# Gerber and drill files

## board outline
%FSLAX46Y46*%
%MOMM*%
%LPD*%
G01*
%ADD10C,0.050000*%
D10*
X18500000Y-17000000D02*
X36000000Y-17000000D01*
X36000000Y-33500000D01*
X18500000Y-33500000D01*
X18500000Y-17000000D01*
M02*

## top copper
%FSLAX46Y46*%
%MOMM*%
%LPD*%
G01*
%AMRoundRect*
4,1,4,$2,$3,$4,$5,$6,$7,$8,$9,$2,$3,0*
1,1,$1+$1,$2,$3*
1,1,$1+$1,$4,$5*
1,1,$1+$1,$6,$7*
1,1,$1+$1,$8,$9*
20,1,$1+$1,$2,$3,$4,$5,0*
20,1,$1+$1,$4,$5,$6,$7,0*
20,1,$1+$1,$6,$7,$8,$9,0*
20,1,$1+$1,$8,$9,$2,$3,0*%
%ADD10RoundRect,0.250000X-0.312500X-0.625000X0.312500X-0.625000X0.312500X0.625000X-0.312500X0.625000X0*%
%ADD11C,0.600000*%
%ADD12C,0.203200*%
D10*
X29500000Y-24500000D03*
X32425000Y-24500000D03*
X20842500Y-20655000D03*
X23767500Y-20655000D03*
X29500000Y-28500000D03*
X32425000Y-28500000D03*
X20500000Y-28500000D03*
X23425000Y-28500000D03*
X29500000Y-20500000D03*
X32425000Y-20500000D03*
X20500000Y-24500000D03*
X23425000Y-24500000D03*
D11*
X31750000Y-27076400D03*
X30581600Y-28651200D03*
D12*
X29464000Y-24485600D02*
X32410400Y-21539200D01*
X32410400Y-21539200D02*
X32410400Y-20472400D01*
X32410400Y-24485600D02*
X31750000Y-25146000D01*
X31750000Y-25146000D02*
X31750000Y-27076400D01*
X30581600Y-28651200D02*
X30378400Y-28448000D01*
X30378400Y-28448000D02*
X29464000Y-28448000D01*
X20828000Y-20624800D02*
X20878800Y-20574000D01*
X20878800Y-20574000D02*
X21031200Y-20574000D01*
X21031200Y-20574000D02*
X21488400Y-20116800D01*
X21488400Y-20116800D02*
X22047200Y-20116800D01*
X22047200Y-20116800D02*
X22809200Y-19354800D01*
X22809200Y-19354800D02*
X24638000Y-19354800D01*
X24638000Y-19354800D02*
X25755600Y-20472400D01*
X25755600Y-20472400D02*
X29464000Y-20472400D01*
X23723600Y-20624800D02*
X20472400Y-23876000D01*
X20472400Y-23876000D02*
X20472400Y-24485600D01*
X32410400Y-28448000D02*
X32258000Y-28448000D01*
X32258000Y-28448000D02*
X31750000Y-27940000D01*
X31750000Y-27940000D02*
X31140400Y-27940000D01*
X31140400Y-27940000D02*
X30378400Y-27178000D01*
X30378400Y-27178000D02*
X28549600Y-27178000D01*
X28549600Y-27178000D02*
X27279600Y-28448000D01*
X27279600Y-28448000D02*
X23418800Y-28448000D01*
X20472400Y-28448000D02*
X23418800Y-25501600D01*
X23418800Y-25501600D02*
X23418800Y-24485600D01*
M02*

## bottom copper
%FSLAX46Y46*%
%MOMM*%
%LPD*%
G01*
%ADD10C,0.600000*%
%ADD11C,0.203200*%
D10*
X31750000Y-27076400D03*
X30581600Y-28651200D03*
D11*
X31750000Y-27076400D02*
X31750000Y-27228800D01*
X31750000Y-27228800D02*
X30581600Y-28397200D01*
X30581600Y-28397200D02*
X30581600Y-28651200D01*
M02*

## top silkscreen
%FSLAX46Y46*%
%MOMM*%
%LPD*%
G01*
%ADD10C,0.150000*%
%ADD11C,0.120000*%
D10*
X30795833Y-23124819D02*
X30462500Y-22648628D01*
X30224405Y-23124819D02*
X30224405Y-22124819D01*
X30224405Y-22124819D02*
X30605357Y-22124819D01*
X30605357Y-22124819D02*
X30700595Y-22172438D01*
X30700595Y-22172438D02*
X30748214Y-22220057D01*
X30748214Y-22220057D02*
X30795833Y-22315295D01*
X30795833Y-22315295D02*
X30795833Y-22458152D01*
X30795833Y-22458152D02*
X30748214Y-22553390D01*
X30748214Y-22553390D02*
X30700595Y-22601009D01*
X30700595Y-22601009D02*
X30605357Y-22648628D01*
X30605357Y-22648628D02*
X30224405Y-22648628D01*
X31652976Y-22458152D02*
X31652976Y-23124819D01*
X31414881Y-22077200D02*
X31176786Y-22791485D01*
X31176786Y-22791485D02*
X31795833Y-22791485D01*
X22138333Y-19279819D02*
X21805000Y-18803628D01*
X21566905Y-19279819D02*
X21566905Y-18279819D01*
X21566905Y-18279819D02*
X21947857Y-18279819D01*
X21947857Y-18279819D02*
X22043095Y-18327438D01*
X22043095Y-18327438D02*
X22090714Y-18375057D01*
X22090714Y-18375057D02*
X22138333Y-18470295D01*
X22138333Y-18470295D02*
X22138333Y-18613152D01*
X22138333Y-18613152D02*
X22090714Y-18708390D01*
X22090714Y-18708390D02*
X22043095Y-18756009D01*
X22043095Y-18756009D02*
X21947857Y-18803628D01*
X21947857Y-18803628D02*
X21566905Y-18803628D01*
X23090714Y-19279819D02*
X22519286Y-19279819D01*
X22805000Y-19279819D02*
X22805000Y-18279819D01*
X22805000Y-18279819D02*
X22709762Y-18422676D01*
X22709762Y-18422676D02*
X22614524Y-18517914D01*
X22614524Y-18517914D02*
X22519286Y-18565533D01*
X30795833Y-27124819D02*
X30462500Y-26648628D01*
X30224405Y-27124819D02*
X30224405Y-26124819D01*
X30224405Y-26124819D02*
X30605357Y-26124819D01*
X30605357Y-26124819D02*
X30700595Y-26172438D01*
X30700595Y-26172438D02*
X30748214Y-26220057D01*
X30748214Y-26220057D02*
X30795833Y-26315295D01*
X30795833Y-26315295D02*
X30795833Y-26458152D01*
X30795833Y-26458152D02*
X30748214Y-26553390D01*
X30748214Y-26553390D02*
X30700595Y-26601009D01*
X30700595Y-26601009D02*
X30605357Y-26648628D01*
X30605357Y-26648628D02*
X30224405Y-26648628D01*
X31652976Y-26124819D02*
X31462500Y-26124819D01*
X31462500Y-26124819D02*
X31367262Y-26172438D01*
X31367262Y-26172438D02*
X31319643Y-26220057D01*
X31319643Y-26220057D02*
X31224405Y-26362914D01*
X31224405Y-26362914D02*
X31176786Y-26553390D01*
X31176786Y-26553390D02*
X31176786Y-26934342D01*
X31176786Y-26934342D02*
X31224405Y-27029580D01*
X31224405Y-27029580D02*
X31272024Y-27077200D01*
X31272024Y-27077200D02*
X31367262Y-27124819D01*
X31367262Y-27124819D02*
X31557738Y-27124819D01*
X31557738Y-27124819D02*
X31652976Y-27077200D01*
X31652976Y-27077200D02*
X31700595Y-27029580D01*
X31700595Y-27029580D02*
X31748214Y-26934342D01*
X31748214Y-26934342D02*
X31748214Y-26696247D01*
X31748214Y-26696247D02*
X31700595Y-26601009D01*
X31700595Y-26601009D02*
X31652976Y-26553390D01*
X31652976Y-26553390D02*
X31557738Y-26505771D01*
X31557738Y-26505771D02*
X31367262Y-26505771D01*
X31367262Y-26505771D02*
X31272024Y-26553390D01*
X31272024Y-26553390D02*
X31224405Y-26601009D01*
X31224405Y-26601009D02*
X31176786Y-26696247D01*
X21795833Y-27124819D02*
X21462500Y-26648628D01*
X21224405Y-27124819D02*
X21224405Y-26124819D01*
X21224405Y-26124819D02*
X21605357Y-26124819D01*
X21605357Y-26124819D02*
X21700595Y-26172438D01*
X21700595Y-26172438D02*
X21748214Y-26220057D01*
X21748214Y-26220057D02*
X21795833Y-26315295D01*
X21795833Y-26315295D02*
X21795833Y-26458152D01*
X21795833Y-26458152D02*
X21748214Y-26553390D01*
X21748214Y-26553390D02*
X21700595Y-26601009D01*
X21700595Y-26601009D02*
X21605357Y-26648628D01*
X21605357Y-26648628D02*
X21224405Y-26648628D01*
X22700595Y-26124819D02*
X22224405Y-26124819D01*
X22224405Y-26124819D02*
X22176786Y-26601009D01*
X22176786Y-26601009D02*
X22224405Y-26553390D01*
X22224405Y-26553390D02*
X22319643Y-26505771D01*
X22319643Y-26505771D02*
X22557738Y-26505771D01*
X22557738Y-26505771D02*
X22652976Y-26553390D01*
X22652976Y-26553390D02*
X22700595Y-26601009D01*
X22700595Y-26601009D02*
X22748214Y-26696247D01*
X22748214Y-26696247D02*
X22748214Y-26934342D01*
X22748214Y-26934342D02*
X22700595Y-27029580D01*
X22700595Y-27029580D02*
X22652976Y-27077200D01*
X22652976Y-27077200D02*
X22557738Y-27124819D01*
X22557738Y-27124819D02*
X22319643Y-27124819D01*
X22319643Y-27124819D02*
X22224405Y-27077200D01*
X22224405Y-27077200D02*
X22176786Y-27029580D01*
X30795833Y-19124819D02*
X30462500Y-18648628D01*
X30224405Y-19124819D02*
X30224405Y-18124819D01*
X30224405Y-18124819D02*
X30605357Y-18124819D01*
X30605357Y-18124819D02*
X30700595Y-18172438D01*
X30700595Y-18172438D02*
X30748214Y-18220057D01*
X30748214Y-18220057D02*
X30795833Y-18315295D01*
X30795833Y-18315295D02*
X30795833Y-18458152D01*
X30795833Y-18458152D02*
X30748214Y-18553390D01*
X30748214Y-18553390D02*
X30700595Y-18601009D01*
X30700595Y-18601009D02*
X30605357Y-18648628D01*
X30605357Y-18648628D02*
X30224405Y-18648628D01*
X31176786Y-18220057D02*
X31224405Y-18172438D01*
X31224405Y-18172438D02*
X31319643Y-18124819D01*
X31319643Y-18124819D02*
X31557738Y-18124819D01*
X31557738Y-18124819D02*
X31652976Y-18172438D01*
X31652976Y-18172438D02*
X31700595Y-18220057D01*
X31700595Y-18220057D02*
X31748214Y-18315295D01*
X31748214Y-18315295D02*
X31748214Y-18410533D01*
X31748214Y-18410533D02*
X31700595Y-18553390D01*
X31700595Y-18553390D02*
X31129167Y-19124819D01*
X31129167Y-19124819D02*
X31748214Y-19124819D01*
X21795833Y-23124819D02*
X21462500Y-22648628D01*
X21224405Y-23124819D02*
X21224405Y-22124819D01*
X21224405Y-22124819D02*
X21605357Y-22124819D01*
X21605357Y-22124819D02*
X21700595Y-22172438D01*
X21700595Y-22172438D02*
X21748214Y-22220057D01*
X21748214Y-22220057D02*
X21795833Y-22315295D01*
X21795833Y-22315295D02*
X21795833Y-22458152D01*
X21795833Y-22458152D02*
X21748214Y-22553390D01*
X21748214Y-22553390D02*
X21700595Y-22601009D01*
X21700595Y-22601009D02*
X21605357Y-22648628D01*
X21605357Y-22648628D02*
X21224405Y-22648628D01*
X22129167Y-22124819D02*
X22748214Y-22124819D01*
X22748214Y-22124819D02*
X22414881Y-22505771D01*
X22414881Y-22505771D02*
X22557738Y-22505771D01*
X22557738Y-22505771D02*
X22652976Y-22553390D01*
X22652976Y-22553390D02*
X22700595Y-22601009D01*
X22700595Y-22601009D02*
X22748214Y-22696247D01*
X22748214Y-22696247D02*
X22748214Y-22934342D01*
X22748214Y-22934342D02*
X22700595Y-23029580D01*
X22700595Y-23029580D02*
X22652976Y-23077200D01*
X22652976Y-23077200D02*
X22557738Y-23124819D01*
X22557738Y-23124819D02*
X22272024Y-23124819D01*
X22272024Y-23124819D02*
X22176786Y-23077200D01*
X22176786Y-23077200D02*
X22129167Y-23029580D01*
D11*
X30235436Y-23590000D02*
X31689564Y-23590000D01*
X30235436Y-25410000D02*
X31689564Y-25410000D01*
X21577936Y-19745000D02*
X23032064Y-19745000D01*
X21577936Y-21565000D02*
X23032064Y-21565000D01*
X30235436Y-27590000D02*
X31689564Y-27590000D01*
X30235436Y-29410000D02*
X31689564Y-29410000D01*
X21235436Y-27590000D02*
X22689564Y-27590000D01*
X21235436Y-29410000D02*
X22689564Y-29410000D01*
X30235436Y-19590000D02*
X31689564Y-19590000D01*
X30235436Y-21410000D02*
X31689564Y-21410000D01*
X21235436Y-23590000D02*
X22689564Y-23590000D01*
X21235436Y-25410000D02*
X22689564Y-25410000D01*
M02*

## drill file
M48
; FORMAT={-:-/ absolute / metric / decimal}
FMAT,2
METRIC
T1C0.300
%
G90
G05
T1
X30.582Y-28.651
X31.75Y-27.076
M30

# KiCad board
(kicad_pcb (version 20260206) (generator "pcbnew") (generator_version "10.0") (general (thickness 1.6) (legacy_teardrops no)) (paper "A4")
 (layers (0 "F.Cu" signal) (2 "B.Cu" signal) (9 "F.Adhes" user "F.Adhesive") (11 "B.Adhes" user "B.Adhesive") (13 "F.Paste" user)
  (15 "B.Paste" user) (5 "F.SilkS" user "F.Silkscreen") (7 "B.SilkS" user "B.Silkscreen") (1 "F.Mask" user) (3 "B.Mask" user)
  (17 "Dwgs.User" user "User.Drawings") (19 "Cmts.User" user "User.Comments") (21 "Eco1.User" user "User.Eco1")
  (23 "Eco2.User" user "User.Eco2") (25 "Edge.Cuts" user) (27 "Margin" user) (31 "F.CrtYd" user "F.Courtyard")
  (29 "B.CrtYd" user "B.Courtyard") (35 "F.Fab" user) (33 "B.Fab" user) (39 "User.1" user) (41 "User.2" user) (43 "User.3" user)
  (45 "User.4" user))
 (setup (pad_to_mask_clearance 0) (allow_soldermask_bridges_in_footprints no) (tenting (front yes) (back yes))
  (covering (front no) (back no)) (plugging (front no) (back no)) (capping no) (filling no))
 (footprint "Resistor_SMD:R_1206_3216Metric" (layer "F.Cu") (at 30.9625 24.5)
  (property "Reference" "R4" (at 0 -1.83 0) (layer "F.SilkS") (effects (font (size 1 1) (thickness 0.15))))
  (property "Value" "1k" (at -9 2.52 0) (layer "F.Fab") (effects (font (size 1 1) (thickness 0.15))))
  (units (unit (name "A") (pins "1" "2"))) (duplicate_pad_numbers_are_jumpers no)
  (fp_line (start -0.727064 -0.91) (end 0.727064 -0.91) (stroke (width 0.12) (type solid)) (layer "F.SilkS"))
  (fp_line (start -0.727064 0.91) (end 0.727064 0.91) (stroke (width 0.12) (type solid)) (layer "F.SilkS"))
  (pad "1" smd roundrect (at -1.4625 0) (size 1.125 1.75) (layers "F.Cu" "F.Mask" "F.Paste") (roundrect_rratio 0.222222)
   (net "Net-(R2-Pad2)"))
  (pad "2" smd roundrect (at 1.4625 0) (size 1.125 1.75) (layers "F.Cu" "F.Mask" "F.Paste") (roundrect_rratio 0.222222)
   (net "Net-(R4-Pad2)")))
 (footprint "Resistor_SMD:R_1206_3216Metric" (layer "F.Cu") (at 22.305 20.655)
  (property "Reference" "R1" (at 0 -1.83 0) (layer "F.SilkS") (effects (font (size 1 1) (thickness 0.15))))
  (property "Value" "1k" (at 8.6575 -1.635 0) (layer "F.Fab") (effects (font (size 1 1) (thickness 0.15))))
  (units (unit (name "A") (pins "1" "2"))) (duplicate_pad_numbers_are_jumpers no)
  (fp_line (start -0.727064 -0.91) (end 0.727064 -0.91) (stroke (width 0.12) (type solid)) (layer "F.SilkS"))
  (fp_line (start -0.727064 0.91) (end 0.727064 0.91) (stroke (width 0.12) (type solid)) (layer "F.SilkS"))
  (pad "1" smd roundrect (at -1.4625 0) (size 1.125 1.75) (layers "F.Cu" "F.Mask" "F.Paste") (roundrect_rratio 0.222222)
   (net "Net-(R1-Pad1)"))
  (pad "2" smd roundrect (at 1.4625 0) (size 1.125 1.75) (layers "F.Cu" "F.Mask" "F.Paste") (roundrect_rratio 0.222222)
   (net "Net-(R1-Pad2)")))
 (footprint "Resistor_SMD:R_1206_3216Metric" (layer "F.Cu") (at 30.9625 28.5)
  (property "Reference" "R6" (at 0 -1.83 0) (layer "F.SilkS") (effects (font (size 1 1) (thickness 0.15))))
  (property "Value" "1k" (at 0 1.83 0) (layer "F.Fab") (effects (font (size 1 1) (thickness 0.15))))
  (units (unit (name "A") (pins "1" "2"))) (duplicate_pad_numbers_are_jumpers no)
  (fp_line (start -0.727064 -0.91) (end 0.727064 -0.91) (stroke (width 0.12) (type solid)) (layer "F.SilkS"))
  (fp_line (start -0.727064 0.91) (end 0.727064 0.91) (stroke (width 0.12) (type solid)) (layer "F.SilkS"))
  (pad "1" smd roundrect (at -1.4625 0) (size 1.125 1.75) (layers "F.Cu" "F.Mask" "F.Paste") (roundrect_rratio 0.222222)
   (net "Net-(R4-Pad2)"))
  (pad "2" smd roundrect (at 1.4625 0) (size 1.125 1.75) (layers "F.Cu" "F.Mask" "F.Paste") (roundrect_rratio 0.222222)
   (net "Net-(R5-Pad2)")))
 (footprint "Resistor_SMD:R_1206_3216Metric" (layer "F.Cu") (at 21.9625 28.5)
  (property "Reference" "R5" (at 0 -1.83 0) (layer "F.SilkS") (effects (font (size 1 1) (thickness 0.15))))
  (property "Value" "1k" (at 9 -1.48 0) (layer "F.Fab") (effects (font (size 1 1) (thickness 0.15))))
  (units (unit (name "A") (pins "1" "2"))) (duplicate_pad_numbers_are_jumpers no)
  (fp_line (start -0.727064 -0.91) (end 0.727064 -0.91) (stroke (width 0.12) (type solid)) (layer "F.SilkS"))
  (fp_line (start -0.727064 0.91) (end 0.727064 0.91) (stroke (width 0.12) (type solid)) (layer "F.SilkS"))
  (pad "1" smd roundrect (at -1.4625 0) (size 1.125 1.75) (layers "F.Cu" "F.Mask" "F.Paste") (roundrect_rratio 0.222222)
   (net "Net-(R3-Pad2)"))
  (pad "2" smd roundrect (at 1.4625 0) (size 1.125 1.75) (layers "F.Cu" "F.Mask" "F.Paste") (roundrect_rratio 0.222222)
   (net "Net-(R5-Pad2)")))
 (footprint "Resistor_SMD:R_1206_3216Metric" (layer "F.Cu") (at 30.9625 20.5)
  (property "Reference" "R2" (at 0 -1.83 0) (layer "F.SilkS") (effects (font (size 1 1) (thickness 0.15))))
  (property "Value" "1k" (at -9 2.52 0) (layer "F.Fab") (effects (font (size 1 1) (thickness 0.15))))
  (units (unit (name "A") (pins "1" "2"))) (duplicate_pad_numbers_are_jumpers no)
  (fp_line (start -0.727064 -0.91) (end 0.727064 -0.91) (stroke (width 0.12) (type solid)) (layer "F.SilkS"))
  (fp_line (start -0.727064 0.91) (end 0.727064 0.91) (stroke (width 0.12) (type solid)) (layer "F.SilkS"))
  (pad "1" smd roundrect (at -1.4625 0) (size 1.125 1.75) (layers "F.Cu" "F.Mask" "F.Paste") (roundrect_rratio 0.222222)
   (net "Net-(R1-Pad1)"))
  (pad "2" smd roundrect (at 1.4625 0) (size 1.125 1.75) (layers "F.Cu" "F.Mask" "F.Paste") (roundrect_rratio 0.222222)
   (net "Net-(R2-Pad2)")))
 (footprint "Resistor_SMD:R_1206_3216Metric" (layer "F.Cu") (at 21.9625 24.5)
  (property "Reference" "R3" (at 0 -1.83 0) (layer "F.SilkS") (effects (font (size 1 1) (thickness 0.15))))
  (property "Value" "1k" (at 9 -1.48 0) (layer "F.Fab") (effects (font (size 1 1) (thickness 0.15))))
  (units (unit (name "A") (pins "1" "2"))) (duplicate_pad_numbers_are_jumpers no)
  (fp_line (start -0.727064 -0.91) (end 0.727064 -0.91) (stroke (width 0.12) (type solid)) (layer "F.SilkS"))
  (fp_line (start -0.727064 0.91) (end 0.727064 0.91) (stroke (width 0.12) (type solid)) (layer "F.SilkS"))
  (pad "1" smd roundrect (at -1.4625 0) (size 1.125 1.75) (layers "F.Cu" "F.Mask" "F.Paste") (roundrect_rratio 0.222222)
   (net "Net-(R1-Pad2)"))
  (pad "2" smd roundrect (at 1.4625 0) (size 1.125 1.75) (layers "F.Cu" "F.Mask" "F.Paste") (roundrect_rratio 0.222222)
   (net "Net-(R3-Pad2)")))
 (gr_rect (start 18.5 17) (end 36 33.5) (stroke (width 0.05) (type default)) (fill no) (layer "Edge.Cuts"))
 (segment (start 29.464 24.4856) (end 32.4104 21.5392) (width 0.2032) (layer "F.Cu") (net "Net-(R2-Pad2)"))
 (segment (start 32.4104 21.5392) (end 32.4104 20.4724) (width 0.2032) (layer "F.Cu") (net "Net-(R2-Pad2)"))
 (segment (start 32.4104 24.4856) (end 31.75 25.146) (width 0.2032) (layer "F.Cu") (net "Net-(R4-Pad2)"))
 (segment (start 31.75 25.146) (end 31.75 27.0764) (width 0.2032) (layer "F.Cu") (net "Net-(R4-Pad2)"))
 (segment (start 30.5816 28.6512) (end 30.3784 28.448) (width 0.2032) (layer "F.Cu") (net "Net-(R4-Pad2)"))
 (segment (start 30.3784 28.448) (end 29.464 28.448) (width 0.2032) (layer "F.Cu") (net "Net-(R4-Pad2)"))
 (segment (start 31.75 27.0764) (end 31.75 27.2288) (width 0.2032) (layer "B.Cu") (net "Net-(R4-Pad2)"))
 (segment (start 31.75 27.2288) (end 30.5816 28.3972) (width 0.2032) (layer "B.Cu") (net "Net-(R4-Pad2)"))
 (segment (start 30.5816 28.3972) (end 30.5816 28.6512) (width 0.2032) (layer "B.Cu") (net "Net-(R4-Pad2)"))
 (via (at 31.75 27.0764) (size 0.6) (drill 0.3) (layers "F.Cu" "B.Cu") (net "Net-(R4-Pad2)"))
 (via (at 30.5816 28.6512) (size 0.6) (drill 0.3) (layers "F.Cu" "B.Cu") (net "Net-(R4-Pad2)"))
 (segment (start 20.828 20.6248) (end 20.8788 20.574) (width 0.2032) (layer "F.Cu") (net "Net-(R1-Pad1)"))
 (segment (start 20.8788 20.574) (end 21.0312 20.574) (width 0.2032) (layer "F.Cu") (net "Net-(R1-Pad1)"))
 (segment (start 21.0312 20.574) (end 21.4884 20.1168) (width 0.2032) (layer "F.Cu") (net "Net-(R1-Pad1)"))
 (segment (start 21.4884 20.1168) (end 22.0472 20.1168) (width 0.2032) (layer "F.Cu") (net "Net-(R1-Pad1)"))
 (segment (start 22.0472 20.1168) (end 22.8092 19.3548) (width 0.2032) (layer "F.Cu") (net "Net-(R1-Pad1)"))
 (segment (start 22.8092 19.3548) (end 24.638 19.3548) (width 0.2032) (layer "F.Cu") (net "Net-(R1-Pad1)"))
 (segment (start 24.638 19.3548) (end 25.7556 20.4724) (width 0.2032) (layer "F.Cu") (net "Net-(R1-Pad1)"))
 (segment (start 25.7556 20.4724) (end 29.464 20.4724) (width 0.2032) (layer "F.Cu") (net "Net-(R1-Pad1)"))
 (segment (start 23.7236 20.6248) (end 20.4724 23.876) (width 0.2032) (layer "F.Cu") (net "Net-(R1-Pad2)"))
 (segment (start 20.4724 23.876) (end 20.4724 24.4856) (width 0.2032) (layer "F.Cu") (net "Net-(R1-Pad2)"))
 (segment (start 32.4104 28.448) (end 32.258 28.448) (width 0.2032) (layer "F.Cu") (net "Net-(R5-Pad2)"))
 (segment (start 32.258 28.448) (end 31.75 27.94) (width 0.2032) (layer "F.Cu") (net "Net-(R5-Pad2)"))
 (segment (start 31.75 27.94) (end 31.1404 27.94) (width 0.2032) (layer "F.Cu") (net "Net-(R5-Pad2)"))
 (segment (start 31.1404 27.94) (end 30.3784 27.178) (width 0.2032) (layer "F.Cu") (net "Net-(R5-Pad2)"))
 (segment (start 30.3784 27.178) (end 28.5496 27.178) (width 0.2032) (layer "F.Cu") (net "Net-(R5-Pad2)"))
 (segment (start 28.5496 27.178) (end 27.2796 28.448) (width 0.2032) (layer "F.Cu") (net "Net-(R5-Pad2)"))
 (segment (start 27.2796 28.448) (end 23.4188 28.448) (width 0.2032) (layer "F.Cu") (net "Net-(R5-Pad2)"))
 (segment (start 20.4724 28.448) (end 23.4188 25.5016) (width 0.2032) (layer "F.Cu") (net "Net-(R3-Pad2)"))
 (segment (start 23.4188 25.5016) (end 23.4188 24.4856) (width 0.2032) (layer "F.Cu") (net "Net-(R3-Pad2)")))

